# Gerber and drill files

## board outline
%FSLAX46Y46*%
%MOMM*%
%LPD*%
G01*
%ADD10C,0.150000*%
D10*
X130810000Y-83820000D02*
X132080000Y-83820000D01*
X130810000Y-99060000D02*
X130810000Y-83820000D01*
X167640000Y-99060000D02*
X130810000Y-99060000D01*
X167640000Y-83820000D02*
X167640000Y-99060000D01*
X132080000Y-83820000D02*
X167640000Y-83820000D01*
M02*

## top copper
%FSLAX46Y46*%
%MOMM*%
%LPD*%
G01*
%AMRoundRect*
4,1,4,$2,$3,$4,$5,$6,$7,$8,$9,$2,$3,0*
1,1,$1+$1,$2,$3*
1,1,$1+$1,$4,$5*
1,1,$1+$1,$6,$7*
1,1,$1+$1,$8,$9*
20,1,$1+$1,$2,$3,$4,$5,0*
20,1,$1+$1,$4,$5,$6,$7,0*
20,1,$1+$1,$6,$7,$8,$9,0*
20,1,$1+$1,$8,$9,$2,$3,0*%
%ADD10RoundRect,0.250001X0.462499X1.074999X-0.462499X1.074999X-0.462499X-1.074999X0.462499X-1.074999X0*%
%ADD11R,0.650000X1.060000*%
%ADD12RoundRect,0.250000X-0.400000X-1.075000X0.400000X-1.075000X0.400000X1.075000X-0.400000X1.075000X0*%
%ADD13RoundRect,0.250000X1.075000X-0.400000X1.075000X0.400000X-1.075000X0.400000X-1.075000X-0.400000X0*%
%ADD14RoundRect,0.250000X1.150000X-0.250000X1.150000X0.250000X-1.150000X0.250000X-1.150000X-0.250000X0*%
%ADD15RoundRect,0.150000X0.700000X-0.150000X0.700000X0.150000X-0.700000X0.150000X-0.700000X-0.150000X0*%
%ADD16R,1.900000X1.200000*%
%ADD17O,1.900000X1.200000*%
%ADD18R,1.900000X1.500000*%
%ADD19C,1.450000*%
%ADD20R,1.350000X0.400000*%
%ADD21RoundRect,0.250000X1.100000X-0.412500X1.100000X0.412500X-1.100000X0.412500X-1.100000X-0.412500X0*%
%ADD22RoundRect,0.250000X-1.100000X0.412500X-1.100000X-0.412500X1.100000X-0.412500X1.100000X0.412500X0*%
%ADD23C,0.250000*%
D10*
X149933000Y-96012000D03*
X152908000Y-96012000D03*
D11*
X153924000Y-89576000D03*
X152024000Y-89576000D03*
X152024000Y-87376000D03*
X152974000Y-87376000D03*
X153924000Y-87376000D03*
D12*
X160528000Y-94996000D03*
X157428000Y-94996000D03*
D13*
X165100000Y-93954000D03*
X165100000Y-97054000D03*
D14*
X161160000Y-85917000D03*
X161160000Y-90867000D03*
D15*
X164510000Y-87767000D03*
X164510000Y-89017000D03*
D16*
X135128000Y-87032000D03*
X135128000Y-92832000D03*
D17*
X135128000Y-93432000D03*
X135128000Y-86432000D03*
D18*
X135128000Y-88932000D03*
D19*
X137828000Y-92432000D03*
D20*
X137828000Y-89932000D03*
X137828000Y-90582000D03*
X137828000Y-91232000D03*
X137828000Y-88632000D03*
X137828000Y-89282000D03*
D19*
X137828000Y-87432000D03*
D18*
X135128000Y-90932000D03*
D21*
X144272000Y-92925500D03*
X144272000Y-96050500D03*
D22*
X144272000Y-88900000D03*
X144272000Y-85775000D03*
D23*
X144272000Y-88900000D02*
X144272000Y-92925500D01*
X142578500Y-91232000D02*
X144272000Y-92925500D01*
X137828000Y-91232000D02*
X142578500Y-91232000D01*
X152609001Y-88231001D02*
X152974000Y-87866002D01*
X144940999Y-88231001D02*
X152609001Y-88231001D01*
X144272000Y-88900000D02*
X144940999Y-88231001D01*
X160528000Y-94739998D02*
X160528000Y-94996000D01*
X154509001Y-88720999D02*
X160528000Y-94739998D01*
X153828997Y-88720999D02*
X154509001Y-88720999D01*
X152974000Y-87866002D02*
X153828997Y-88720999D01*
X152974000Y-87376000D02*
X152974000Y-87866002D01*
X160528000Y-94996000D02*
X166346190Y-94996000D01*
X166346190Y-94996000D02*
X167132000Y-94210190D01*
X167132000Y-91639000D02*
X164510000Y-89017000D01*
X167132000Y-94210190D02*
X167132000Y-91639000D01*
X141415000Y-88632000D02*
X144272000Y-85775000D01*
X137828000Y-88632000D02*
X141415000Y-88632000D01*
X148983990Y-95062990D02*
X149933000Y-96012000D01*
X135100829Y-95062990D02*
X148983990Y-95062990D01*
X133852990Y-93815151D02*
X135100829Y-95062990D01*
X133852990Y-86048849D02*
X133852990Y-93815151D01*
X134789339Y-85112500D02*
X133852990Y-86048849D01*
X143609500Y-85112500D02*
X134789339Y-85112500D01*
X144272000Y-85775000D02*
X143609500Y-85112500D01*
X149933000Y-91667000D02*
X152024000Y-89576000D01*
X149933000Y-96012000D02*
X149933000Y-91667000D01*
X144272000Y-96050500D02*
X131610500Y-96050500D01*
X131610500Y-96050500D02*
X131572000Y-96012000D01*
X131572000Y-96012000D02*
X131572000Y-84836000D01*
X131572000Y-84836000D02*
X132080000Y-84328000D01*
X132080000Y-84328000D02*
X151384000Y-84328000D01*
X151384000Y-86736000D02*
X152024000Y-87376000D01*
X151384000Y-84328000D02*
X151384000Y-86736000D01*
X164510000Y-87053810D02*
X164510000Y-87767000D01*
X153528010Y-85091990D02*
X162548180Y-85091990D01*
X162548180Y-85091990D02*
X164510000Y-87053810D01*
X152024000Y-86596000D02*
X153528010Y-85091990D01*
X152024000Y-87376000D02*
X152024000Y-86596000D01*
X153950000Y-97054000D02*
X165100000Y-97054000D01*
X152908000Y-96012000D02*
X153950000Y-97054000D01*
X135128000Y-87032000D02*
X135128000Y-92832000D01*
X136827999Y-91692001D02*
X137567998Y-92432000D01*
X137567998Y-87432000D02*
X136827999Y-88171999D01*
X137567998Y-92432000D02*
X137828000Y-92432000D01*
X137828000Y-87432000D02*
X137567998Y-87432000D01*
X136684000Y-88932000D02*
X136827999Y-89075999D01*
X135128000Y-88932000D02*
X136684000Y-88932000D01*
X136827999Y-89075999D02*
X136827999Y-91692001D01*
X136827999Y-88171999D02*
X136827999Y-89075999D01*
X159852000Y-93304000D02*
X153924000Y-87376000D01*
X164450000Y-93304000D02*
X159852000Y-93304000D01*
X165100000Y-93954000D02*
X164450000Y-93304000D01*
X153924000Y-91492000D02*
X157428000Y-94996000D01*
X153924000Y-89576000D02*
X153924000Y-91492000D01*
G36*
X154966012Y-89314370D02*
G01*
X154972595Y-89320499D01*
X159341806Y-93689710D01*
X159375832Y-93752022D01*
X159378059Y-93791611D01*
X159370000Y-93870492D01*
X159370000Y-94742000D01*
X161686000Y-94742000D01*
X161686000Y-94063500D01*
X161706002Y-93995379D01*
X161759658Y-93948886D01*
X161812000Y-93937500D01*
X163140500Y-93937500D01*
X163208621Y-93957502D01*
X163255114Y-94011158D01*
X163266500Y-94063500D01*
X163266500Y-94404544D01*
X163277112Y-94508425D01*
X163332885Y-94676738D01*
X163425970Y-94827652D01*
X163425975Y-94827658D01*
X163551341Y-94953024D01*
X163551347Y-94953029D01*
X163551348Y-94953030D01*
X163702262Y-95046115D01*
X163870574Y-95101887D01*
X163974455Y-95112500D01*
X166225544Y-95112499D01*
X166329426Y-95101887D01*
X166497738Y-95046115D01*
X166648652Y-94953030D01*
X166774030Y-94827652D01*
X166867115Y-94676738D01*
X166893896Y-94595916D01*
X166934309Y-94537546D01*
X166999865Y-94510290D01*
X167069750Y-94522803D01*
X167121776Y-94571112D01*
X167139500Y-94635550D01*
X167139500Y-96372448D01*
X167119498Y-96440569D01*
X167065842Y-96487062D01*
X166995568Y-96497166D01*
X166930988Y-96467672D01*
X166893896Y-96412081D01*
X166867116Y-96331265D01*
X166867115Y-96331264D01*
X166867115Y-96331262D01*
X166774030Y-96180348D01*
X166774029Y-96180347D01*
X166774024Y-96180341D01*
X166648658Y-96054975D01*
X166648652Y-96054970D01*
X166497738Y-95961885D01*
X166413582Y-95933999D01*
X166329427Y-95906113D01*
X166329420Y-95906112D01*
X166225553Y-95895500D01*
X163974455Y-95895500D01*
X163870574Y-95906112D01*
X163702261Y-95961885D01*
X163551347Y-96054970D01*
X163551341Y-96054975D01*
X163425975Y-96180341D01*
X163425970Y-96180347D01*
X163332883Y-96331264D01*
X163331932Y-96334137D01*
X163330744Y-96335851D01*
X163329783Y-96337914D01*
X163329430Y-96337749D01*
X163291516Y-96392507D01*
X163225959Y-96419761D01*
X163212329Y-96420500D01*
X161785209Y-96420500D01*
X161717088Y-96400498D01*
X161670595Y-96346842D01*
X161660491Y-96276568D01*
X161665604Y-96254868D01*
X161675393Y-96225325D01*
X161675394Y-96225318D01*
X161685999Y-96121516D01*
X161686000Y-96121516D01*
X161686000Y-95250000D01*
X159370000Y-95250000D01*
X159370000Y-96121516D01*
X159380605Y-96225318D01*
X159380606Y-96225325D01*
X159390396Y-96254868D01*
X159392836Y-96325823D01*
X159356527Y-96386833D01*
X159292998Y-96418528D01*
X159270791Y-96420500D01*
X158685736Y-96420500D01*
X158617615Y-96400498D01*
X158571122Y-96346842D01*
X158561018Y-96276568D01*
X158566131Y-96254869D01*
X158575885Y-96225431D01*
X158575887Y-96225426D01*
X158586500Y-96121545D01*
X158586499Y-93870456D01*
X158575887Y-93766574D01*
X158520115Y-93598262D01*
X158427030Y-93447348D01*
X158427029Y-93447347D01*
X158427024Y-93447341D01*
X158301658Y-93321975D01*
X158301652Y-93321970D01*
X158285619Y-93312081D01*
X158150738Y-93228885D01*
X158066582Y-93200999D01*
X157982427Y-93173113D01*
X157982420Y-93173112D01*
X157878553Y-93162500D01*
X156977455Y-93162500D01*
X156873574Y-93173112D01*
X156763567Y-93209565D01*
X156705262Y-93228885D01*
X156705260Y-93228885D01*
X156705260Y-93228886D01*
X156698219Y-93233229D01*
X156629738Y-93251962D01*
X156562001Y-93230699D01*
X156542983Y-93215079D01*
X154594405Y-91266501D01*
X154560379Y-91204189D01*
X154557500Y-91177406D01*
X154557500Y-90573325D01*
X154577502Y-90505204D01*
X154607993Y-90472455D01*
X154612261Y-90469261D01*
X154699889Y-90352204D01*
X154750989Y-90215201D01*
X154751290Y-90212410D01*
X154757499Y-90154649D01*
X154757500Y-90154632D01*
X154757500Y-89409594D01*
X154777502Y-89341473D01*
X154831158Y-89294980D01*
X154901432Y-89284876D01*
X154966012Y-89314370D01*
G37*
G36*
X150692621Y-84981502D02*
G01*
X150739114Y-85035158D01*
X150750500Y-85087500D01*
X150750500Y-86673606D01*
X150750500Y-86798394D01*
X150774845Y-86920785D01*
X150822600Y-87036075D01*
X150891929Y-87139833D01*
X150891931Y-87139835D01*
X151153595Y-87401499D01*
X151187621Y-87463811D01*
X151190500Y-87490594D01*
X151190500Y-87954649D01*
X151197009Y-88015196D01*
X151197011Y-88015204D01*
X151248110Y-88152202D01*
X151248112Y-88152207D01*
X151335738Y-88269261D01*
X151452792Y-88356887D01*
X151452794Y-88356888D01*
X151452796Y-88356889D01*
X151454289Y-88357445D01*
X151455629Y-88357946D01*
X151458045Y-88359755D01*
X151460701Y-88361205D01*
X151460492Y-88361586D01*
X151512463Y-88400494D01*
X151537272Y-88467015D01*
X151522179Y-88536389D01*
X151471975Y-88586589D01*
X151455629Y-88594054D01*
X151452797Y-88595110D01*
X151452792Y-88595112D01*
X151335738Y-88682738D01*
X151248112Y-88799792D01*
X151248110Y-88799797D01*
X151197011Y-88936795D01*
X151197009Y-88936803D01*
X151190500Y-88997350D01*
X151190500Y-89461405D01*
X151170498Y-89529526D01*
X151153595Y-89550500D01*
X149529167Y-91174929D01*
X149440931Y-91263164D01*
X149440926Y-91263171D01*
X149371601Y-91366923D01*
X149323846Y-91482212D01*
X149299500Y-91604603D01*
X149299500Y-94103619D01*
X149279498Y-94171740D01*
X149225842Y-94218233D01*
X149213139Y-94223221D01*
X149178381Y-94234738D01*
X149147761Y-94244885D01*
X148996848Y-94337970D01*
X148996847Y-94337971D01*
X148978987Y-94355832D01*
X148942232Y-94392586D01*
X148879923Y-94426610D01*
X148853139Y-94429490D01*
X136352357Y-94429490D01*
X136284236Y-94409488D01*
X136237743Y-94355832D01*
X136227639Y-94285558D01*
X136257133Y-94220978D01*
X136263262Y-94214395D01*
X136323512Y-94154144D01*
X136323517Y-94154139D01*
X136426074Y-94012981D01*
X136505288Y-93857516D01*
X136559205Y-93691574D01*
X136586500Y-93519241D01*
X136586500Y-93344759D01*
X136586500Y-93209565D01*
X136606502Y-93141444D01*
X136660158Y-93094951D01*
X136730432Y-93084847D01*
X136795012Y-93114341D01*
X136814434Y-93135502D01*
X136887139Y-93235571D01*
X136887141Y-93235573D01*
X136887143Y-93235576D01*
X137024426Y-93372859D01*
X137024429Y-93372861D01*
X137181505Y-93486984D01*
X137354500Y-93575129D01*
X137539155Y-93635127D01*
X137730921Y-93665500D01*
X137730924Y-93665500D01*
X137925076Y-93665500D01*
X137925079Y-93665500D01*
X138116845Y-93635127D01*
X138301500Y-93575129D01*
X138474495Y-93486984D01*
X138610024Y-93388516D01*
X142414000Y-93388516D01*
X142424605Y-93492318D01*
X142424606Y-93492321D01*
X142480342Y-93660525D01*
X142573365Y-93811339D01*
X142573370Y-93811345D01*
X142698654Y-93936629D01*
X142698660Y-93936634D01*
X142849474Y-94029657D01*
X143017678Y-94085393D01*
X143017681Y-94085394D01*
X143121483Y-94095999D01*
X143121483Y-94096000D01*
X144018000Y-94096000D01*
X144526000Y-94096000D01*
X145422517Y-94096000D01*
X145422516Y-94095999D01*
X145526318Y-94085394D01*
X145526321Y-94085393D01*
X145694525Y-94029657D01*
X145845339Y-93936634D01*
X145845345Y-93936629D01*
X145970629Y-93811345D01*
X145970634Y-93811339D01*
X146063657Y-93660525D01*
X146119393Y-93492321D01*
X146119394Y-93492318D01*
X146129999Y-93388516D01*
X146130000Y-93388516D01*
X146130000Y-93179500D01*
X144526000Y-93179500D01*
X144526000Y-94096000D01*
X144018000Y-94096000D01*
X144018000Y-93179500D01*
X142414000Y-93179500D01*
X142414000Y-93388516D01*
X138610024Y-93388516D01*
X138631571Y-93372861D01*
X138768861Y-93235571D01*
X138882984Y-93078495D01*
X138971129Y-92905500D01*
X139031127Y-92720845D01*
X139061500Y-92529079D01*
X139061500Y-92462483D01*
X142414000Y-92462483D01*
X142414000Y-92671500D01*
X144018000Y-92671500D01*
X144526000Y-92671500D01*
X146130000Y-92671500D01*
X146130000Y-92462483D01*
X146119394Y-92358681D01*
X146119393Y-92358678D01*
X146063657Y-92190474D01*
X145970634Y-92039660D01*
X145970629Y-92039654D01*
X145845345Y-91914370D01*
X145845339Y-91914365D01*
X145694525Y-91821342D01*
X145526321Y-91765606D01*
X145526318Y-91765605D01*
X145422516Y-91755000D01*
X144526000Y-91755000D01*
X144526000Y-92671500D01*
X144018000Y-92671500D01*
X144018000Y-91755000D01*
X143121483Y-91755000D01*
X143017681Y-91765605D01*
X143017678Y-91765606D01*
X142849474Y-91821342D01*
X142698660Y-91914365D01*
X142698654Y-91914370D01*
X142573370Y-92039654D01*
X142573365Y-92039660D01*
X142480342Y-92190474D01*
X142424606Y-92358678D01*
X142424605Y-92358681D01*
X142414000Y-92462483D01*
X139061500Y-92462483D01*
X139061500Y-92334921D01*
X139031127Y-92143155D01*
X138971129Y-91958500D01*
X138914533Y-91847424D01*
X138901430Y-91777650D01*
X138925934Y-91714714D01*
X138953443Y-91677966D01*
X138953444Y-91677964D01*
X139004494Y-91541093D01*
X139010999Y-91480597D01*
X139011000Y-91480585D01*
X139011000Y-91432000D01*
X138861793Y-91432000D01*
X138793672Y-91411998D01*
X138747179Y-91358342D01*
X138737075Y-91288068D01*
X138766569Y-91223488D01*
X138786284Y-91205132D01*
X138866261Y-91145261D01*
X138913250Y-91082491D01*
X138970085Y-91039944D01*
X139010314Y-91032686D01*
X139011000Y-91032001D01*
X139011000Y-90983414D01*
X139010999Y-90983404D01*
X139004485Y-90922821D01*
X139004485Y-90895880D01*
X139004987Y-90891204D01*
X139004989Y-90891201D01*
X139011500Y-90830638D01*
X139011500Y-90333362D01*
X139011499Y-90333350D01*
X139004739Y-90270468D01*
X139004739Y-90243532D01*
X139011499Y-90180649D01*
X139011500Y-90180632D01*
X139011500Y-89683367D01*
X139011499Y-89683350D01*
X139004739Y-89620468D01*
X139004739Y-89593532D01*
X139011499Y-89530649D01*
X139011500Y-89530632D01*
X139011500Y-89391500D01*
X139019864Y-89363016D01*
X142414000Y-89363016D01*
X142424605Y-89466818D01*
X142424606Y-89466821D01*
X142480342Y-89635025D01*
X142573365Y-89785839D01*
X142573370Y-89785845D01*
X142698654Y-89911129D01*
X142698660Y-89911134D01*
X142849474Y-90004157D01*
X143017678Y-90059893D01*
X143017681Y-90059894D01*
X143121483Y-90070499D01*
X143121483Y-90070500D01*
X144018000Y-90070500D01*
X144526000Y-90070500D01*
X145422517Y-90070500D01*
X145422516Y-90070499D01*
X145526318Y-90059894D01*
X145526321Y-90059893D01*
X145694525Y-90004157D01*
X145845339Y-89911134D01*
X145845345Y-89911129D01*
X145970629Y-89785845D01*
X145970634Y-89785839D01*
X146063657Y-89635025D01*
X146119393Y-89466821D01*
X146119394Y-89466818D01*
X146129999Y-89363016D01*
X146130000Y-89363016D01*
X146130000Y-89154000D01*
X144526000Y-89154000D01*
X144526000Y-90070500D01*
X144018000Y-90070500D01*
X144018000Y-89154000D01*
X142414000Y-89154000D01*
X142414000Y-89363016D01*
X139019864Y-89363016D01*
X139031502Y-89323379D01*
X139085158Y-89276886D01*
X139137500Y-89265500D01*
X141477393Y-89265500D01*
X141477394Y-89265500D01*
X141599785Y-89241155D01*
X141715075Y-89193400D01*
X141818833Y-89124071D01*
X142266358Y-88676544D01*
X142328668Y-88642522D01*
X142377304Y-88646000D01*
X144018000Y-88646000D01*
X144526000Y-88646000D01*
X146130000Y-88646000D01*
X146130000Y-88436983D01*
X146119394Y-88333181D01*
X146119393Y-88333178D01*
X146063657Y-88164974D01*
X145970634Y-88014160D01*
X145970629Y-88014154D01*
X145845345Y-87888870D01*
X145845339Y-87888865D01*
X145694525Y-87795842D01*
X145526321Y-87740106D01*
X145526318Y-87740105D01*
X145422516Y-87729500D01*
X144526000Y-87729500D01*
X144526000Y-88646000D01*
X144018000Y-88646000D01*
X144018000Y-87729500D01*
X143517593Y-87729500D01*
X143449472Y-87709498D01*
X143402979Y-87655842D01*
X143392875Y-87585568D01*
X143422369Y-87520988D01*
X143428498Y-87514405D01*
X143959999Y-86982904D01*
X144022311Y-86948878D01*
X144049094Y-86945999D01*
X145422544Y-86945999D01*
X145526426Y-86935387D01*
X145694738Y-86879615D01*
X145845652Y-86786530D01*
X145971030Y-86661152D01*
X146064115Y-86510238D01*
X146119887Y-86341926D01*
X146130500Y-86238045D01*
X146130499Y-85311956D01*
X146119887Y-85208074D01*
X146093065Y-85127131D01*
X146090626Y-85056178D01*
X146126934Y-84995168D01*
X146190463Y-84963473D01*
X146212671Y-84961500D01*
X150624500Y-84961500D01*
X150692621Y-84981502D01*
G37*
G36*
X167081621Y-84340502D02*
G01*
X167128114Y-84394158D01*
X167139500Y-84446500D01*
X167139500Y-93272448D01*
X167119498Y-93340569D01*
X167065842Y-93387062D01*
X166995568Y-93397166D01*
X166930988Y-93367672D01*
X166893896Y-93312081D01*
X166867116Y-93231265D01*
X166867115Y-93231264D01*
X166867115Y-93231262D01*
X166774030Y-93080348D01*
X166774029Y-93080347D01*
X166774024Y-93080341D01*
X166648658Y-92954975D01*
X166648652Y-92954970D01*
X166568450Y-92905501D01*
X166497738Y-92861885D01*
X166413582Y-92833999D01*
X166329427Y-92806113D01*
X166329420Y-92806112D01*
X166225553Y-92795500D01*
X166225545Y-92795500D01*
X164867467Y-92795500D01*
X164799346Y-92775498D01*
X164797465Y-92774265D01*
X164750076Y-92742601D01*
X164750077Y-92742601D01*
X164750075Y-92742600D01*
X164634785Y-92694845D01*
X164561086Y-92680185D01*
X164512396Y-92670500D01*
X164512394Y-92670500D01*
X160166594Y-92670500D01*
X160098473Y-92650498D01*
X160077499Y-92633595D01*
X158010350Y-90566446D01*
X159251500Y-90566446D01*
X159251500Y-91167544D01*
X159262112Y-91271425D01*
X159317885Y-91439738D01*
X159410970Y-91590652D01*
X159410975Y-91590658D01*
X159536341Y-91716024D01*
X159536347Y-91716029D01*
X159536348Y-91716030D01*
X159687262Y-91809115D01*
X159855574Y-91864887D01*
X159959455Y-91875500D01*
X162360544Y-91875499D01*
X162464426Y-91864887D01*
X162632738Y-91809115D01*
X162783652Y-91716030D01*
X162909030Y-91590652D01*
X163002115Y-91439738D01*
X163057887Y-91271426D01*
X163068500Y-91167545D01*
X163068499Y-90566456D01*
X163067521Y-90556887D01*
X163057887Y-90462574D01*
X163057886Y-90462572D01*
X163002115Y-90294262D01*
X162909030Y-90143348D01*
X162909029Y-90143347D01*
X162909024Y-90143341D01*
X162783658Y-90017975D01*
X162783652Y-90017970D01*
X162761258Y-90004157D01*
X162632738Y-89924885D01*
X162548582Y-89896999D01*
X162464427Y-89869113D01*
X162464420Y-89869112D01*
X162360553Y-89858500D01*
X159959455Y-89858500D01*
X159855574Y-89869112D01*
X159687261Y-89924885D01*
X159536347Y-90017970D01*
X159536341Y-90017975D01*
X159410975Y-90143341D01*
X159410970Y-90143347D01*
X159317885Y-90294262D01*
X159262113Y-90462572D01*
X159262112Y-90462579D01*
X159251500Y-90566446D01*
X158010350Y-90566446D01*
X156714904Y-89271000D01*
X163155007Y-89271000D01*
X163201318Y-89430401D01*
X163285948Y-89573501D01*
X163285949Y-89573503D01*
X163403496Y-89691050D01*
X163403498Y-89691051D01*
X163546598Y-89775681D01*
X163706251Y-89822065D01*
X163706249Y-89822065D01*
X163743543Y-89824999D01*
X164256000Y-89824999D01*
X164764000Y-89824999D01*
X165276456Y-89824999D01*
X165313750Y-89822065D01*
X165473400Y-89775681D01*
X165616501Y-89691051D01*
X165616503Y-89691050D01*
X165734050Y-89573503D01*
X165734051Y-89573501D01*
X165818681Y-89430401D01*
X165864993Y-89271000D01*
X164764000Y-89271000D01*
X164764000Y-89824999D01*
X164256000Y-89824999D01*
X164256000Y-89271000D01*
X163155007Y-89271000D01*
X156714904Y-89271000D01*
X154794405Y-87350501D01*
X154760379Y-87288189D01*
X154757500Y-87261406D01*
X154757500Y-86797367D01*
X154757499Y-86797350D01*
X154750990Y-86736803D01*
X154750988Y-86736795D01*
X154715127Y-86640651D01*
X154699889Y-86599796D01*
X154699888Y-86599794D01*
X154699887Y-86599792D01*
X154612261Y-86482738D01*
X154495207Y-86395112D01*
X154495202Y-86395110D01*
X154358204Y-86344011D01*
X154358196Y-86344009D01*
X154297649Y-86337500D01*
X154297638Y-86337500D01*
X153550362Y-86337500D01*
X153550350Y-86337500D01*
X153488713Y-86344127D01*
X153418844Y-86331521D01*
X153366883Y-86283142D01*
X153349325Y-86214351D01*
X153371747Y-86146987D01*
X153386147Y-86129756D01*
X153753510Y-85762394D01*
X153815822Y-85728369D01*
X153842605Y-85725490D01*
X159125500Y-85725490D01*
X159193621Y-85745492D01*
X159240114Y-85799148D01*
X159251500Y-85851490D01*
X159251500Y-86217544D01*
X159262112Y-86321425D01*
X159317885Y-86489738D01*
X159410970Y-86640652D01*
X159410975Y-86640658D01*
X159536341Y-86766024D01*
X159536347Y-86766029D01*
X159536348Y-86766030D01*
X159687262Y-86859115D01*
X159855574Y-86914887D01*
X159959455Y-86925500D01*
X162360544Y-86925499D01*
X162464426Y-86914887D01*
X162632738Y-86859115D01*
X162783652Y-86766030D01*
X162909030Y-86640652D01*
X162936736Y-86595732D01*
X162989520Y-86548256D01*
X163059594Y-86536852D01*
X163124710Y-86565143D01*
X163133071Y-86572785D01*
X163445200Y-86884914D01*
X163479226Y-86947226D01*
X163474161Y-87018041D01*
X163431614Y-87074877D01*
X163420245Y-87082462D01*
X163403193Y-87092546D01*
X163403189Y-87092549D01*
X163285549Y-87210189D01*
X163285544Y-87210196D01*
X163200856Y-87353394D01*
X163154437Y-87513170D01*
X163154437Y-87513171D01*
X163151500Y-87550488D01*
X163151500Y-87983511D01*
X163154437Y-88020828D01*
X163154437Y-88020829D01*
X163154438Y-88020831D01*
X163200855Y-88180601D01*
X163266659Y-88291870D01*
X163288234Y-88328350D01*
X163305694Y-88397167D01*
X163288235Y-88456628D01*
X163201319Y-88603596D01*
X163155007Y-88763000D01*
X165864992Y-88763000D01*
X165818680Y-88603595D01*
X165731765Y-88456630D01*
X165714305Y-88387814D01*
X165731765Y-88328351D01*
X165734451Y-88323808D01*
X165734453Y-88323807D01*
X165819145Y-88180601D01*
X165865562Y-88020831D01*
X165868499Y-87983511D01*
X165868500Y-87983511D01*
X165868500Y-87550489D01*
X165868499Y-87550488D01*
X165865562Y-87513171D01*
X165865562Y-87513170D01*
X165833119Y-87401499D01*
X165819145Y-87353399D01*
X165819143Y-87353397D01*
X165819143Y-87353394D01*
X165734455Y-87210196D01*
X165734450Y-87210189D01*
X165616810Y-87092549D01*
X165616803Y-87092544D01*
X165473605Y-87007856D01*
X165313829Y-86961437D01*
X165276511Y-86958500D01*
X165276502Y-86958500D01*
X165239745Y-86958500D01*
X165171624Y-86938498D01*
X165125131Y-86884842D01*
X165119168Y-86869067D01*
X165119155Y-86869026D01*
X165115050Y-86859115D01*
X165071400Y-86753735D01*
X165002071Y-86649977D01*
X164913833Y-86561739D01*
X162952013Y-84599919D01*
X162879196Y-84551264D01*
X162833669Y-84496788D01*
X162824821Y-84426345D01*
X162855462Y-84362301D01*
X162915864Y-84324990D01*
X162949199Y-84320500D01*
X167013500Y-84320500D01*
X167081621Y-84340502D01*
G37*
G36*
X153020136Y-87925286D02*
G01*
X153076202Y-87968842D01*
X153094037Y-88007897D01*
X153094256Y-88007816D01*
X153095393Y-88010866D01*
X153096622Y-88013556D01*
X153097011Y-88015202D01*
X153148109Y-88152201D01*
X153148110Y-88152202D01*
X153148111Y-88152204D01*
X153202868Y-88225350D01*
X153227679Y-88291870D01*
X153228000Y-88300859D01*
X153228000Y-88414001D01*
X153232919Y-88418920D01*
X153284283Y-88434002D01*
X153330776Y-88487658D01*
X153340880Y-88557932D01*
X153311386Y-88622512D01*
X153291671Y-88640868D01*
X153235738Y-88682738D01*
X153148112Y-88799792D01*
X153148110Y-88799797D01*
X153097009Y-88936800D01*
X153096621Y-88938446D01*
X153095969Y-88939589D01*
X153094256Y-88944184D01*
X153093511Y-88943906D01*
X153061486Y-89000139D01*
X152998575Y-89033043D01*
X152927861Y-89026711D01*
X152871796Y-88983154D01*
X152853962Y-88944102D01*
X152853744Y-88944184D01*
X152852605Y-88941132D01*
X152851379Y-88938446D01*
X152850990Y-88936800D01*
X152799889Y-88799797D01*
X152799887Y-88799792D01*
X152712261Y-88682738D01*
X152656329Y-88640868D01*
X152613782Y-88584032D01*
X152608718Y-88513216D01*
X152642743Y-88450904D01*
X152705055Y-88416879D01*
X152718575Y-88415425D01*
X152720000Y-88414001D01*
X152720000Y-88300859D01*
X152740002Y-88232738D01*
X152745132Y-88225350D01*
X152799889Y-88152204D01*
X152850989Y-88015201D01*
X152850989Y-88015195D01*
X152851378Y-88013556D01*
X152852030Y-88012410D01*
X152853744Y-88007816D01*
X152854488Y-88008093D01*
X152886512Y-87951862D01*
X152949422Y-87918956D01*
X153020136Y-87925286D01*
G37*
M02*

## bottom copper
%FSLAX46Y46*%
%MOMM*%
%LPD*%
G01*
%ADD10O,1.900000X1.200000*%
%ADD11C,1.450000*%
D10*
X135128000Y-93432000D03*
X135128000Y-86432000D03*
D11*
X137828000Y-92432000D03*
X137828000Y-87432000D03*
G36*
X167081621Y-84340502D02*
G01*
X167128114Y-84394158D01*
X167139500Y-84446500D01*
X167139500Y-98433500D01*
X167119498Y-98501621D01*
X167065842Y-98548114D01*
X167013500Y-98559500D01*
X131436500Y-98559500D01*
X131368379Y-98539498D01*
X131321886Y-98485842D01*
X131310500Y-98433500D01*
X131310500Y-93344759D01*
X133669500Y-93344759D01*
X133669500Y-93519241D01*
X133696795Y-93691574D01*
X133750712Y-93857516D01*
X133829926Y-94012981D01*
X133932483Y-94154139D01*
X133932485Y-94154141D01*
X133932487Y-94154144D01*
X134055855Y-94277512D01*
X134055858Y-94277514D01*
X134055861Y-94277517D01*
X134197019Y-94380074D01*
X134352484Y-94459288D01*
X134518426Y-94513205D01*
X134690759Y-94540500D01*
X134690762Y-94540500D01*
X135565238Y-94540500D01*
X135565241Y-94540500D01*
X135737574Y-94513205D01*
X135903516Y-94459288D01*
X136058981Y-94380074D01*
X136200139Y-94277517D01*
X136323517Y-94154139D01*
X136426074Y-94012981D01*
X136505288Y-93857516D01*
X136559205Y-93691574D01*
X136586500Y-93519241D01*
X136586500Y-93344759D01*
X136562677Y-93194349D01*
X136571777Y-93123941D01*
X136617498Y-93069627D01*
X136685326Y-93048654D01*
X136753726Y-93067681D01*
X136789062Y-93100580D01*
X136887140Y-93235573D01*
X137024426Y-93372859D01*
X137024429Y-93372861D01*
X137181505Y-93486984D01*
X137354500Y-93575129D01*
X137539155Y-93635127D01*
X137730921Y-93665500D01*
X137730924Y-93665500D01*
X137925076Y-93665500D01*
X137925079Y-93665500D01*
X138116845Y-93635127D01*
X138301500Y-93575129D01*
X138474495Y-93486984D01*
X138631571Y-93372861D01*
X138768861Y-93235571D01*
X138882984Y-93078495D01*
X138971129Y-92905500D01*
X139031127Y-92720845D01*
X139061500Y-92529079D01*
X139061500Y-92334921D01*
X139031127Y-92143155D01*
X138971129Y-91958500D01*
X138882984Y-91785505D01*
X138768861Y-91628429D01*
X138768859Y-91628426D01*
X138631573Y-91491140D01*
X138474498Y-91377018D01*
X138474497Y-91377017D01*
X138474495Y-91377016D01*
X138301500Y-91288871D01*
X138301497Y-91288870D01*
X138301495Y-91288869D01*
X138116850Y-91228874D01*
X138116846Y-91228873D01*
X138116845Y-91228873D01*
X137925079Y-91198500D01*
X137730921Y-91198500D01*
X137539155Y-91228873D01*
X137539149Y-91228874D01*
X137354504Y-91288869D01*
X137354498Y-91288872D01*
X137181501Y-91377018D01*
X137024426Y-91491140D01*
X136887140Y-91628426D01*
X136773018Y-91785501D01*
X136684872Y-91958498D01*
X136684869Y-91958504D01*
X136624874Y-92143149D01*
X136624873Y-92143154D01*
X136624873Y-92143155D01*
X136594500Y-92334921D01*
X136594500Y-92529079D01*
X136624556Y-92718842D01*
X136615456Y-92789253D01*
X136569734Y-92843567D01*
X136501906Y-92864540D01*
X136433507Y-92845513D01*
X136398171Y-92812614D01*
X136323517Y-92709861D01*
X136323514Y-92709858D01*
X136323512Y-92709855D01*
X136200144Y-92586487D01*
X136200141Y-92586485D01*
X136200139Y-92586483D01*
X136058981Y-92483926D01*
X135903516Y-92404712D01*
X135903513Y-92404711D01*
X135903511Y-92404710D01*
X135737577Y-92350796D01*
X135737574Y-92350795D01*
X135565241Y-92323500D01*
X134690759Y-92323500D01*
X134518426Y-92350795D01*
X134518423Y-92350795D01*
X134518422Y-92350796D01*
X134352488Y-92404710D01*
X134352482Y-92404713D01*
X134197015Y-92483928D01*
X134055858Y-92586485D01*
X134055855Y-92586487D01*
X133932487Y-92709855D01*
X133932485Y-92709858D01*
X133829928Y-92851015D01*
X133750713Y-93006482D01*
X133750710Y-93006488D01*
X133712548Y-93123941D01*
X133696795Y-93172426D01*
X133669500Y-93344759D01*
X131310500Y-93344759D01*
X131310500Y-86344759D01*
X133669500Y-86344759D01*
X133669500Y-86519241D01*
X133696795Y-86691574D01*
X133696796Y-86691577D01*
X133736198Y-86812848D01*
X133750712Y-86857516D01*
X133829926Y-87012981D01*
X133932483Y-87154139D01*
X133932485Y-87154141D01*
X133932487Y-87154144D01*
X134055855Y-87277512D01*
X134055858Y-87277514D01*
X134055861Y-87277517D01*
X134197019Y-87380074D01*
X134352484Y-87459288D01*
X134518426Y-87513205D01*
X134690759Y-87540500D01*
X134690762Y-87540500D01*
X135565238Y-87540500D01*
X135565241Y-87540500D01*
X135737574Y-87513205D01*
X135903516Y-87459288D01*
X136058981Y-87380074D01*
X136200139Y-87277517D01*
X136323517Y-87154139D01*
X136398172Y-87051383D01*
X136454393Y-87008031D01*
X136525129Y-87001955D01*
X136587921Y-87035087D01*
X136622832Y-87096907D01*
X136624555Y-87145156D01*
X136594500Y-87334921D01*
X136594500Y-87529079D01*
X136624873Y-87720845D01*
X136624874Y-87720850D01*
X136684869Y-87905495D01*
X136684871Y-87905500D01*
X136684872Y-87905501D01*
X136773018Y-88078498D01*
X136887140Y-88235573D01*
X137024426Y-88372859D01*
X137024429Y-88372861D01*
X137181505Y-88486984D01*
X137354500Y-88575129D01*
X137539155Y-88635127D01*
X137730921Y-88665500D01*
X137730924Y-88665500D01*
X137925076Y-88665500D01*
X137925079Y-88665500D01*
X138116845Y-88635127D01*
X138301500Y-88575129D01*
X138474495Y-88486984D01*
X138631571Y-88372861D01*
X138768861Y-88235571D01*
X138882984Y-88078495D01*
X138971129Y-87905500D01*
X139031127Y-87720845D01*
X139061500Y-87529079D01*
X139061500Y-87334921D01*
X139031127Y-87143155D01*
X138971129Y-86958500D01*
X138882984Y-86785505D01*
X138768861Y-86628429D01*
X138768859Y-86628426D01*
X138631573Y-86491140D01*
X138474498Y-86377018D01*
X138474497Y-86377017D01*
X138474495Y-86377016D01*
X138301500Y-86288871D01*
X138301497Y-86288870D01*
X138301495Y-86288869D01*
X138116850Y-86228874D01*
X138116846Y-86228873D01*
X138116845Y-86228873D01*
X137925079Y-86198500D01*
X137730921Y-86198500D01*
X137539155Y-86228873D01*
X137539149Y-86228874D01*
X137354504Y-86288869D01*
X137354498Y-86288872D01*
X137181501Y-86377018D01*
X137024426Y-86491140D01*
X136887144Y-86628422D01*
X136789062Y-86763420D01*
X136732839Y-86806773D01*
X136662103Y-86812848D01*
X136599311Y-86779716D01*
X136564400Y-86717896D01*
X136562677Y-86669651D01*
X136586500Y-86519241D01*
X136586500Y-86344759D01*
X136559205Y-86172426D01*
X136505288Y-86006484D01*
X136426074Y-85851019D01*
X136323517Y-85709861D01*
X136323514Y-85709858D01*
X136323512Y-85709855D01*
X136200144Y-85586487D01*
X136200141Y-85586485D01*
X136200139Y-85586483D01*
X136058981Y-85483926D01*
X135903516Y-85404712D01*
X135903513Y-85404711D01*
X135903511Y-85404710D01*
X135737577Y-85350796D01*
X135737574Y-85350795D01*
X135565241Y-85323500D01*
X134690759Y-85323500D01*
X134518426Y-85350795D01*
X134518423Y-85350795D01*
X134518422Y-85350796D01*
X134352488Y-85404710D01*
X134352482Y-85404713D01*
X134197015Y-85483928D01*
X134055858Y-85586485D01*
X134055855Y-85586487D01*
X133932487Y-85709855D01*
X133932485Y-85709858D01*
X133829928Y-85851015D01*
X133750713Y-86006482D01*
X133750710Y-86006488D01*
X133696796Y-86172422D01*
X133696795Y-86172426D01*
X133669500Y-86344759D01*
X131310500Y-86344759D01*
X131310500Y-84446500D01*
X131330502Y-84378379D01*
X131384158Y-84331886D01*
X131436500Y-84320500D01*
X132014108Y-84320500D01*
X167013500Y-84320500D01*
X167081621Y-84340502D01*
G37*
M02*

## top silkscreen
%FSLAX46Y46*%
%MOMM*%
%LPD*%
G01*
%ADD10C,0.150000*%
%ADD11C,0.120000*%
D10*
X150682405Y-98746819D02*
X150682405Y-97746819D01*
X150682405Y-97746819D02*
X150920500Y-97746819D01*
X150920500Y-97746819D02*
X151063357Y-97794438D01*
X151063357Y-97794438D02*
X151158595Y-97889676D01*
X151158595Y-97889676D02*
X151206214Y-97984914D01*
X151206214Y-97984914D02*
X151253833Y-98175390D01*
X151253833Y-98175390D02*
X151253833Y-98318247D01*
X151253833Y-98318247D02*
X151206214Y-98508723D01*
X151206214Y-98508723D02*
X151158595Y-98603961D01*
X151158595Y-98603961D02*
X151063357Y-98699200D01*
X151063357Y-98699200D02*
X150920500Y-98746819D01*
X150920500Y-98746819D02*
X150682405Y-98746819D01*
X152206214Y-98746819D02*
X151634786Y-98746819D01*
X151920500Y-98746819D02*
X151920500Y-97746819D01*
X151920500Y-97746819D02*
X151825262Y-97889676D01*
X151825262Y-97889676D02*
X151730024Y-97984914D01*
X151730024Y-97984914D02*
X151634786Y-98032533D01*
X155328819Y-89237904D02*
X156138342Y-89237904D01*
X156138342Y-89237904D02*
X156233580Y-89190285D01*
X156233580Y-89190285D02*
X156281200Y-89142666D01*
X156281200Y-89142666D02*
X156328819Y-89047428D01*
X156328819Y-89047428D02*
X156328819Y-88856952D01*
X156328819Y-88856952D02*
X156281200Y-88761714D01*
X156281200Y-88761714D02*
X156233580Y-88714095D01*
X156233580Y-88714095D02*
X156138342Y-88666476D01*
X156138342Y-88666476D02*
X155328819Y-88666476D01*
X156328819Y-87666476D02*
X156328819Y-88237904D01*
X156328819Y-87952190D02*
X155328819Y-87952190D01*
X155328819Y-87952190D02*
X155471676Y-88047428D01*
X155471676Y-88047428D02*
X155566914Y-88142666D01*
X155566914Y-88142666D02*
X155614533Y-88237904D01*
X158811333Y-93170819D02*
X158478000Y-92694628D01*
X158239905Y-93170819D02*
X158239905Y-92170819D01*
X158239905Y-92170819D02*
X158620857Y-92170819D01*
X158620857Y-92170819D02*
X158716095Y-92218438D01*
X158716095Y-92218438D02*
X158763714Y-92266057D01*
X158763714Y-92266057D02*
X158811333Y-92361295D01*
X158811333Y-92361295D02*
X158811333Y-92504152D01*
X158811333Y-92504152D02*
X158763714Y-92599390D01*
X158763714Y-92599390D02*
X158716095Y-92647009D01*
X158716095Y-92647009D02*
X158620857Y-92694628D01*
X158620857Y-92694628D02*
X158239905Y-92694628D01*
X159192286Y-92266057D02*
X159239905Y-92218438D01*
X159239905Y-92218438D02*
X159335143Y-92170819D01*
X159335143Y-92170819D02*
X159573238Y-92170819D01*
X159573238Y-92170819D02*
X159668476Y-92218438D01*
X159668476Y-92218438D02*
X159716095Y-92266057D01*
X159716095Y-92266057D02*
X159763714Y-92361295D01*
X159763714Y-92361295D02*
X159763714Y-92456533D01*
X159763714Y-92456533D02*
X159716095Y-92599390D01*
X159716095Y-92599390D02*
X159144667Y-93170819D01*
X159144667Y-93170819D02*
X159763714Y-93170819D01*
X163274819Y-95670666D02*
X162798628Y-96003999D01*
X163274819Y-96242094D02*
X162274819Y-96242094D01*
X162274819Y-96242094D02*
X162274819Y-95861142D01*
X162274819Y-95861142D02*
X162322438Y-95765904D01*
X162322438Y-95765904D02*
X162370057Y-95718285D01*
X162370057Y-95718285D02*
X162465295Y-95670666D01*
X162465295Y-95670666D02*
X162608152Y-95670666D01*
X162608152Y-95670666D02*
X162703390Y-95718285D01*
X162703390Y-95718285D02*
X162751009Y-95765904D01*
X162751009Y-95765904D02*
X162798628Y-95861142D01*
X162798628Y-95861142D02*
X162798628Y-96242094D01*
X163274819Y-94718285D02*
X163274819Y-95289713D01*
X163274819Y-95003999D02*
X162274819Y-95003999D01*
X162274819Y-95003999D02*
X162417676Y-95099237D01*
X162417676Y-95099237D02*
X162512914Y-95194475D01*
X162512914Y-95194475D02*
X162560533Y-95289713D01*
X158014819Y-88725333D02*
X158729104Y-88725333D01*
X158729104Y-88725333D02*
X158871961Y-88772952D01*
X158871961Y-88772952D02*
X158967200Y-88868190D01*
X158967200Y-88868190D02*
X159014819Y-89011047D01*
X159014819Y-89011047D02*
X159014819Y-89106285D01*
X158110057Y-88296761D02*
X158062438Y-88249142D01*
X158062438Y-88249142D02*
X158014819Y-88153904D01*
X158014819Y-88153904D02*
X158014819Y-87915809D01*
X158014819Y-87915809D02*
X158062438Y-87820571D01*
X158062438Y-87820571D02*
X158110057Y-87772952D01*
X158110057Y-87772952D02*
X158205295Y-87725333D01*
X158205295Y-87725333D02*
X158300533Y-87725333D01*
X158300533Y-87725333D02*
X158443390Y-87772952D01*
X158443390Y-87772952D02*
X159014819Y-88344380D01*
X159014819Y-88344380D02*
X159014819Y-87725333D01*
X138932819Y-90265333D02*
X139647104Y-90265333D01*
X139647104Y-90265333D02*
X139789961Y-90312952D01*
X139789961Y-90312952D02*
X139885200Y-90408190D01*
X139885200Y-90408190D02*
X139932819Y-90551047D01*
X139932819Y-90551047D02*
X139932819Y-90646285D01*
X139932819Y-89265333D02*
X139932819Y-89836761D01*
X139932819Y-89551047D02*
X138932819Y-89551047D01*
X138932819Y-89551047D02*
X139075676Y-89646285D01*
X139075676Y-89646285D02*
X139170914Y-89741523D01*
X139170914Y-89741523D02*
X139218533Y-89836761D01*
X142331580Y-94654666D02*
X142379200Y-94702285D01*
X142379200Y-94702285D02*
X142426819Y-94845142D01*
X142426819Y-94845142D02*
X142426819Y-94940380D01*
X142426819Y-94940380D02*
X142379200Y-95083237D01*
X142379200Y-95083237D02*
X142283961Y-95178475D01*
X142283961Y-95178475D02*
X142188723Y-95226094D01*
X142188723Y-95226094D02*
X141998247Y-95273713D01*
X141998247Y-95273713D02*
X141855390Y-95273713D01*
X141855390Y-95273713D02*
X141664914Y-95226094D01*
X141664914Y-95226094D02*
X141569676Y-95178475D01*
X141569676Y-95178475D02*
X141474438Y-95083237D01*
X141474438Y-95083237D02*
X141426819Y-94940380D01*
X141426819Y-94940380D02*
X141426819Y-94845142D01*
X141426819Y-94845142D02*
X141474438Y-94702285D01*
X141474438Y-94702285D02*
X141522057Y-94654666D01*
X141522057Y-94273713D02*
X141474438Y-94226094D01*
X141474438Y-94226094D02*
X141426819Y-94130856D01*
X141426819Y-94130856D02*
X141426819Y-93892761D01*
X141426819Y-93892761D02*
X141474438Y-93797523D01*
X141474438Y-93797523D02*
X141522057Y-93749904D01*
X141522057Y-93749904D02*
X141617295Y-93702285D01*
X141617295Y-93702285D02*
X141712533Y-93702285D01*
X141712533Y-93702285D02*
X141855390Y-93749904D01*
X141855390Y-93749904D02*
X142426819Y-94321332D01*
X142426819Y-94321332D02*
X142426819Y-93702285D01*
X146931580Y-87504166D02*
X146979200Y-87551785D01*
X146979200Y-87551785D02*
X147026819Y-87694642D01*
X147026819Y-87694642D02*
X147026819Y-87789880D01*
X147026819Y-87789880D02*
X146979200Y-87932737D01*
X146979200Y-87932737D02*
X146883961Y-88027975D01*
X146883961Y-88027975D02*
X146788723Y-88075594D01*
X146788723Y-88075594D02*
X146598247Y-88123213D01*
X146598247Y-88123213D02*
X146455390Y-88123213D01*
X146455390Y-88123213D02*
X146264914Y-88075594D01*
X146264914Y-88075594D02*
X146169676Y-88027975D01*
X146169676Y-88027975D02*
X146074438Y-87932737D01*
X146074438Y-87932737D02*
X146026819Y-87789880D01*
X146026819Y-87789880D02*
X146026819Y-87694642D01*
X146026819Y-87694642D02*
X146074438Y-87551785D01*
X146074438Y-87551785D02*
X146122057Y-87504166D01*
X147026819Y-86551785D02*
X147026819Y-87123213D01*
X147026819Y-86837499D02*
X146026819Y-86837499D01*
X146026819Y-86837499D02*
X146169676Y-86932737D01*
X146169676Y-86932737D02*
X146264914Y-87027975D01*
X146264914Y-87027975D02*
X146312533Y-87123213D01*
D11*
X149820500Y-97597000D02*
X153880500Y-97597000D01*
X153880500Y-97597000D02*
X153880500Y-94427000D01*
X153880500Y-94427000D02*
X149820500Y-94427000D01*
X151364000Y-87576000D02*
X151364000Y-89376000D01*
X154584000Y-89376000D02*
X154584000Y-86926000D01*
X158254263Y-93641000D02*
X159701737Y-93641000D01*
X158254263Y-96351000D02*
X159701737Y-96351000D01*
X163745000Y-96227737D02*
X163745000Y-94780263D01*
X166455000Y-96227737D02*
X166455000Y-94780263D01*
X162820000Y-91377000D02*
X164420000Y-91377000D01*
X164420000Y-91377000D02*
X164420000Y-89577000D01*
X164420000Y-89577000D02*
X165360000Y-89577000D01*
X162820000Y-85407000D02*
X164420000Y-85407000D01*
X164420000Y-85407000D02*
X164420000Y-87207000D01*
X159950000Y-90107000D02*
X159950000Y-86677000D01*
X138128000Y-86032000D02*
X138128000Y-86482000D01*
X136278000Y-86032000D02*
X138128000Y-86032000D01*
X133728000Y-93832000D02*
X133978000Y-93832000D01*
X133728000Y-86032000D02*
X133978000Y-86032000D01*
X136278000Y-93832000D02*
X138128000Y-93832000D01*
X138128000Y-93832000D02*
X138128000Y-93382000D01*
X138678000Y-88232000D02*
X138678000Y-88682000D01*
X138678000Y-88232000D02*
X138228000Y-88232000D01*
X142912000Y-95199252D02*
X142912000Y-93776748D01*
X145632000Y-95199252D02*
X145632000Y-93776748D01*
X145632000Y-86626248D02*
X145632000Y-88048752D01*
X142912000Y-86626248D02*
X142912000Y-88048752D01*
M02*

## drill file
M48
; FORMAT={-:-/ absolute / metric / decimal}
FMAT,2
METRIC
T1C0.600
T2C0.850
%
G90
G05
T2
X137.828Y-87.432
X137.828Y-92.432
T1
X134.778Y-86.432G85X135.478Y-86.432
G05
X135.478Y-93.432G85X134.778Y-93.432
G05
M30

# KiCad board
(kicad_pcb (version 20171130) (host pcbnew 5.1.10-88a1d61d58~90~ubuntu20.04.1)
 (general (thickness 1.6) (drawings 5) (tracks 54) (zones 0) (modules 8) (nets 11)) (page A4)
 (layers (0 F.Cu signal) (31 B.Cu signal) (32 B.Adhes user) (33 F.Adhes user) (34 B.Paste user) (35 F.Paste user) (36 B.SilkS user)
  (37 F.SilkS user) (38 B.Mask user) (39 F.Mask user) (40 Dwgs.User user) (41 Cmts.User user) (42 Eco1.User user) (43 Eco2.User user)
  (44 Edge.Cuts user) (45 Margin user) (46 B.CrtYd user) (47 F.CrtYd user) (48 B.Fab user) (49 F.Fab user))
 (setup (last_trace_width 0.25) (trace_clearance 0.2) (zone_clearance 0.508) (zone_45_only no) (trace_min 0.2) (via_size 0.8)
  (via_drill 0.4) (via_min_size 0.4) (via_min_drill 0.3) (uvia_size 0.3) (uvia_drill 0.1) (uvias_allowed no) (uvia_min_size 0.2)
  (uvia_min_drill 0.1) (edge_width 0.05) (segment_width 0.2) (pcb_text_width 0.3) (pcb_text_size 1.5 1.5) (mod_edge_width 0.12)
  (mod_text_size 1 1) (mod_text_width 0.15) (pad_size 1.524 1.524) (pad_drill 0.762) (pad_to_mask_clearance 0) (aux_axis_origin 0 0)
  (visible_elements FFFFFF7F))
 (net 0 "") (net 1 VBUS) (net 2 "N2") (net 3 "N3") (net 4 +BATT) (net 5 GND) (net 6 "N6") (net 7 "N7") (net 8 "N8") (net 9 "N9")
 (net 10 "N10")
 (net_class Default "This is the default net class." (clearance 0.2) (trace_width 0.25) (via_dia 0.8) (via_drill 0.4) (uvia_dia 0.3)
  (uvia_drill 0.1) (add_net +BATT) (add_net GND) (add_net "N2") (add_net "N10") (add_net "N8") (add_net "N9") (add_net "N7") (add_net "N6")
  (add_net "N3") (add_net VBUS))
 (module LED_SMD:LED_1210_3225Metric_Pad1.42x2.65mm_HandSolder (layer F.Cu) (at 151.4205 96.012 180)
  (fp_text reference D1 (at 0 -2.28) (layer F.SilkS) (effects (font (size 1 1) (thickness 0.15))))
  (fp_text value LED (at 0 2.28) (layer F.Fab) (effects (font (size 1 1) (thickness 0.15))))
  (fp_line (start 1.6 -1.585) (end -2.46 -1.585) (layer F.SilkS) (width 0.12))
  (fp_line (start -2.46 -1.585) (end -2.46 1.585) (layer F.SilkS) (width 0.12))
  (fp_line (start -2.46 1.585) (end 1.6 1.585) (layer F.SilkS) (width 0.12))
  (pad 2 smd roundrect (at 1.4875 0 180) (size 1.425 2.65) (layers F.Cu F.Paste F.Mask) (roundrect_rratio 0.175439) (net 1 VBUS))
  (pad 1 smd roundrect (at -1.4875 0 180) (size 1.425 2.65) (layers F.Cu F.Paste F.Mask) (roundrect_rratio 0.175439) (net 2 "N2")))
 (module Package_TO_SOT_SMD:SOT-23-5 (layer F.Cu) (at 152.974 88.476 270)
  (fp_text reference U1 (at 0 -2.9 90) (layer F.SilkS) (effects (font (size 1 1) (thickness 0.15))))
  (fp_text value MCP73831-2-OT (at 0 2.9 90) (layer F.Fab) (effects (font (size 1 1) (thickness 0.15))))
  (fp_line (start -0.9 1.61) (end 0.9 1.61) (layer F.SilkS) (width 0.12))
  (fp_line (start 0.9 -1.61) (end -1.55 -1.61) (layer F.SilkS) (width 0.12))
  (pad 5 smd rect (at 1.1 -0.95 270) (size 1.06 0.65) (layers F.Cu F.Paste F.Mask) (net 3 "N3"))
  (pad 4 smd rect (at 1.1 0.95 270) (size 1.06 0.65) (layers F.Cu F.Paste F.Mask) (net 1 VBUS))
  (pad 3 smd rect (at -1.1 0.95 270) (size 1.06 0.65) (layers F.Cu F.Paste F.Mask) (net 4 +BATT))
  (pad 2 smd rect (at -1.1 0 270) (size 1.06 0.65) (layers F.Cu F.Paste F.Mask) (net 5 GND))
  (pad 1 smd rect (at -1.1 -0.95 270) (size 1.06 0.65) (layers F.Cu F.Paste F.Mask) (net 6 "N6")))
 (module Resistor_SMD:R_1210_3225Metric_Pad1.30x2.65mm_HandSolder (layer F.Cu) (at 158.978 94.996)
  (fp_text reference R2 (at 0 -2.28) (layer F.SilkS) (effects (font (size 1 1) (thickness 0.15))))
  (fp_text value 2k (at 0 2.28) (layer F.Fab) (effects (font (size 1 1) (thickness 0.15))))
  (fp_line (start -0.723737 -1.355) (end 0.723737 -1.355) (layer F.SilkS) (width 0.12))
  (fp_line (start -0.723737 1.355) (end 0.723737 1.355) (layer F.SilkS) (width 0.12))
  (pad 2 smd roundrect (at 1.55 0) (size 1.3 2.65) (layers F.Cu F.Paste F.Mask) (roundrect_rratio 0.192308) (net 5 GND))
  (pad 1 smd roundrect (at -1.55 0) (size 1.3 2.65) (layers F.Cu F.Paste F.Mask) (roundrect_rratio 0.192308) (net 3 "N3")))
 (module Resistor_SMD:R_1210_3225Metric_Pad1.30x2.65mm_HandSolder (layer F.Cu) (at 165.1 95.504 90)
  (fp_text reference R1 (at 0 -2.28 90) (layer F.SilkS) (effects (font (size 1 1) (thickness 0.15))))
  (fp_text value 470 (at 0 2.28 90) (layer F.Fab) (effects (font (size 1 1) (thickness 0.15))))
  (fp_line (start -0.723737 -1.355) (end 0.723737 -1.355) (layer F.SilkS) (width 0.12))
  (fp_line (start -0.723737 1.355) (end 0.723737 1.355) (layer F.SilkS) (width 0.12))
  (pad 2 smd roundrect (at 1.55 0 90) (size 1.3 2.65) (layers F.Cu F.Paste F.Mask) (roundrect_rratio 0.192308) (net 6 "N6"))
  (pad 1 smd roundrect (at -1.55 0 90) (size 1.3 2.65) (layers F.Cu F.Paste F.Mask) (roundrect_rratio 0.192308) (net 2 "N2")))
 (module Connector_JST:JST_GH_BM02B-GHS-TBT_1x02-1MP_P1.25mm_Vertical (layer F.Cu) (at 162.56 88.392 90)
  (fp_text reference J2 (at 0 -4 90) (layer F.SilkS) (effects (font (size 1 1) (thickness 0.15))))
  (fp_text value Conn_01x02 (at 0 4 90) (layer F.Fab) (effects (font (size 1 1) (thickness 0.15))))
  (fp_line (start -2.985 0.26) (end -2.985 1.86) (layer F.SilkS) (width 0.12))
  (fp_line (start -2.985 1.86) (end -1.185 1.86) (layer F.SilkS) (width 0.12))
  (fp_line (start -1.185 1.86) (end -1.185 2.8) (layer F.SilkS) (width 0.12))
  (fp_line (start 2.985 0.26) (end 2.985 1.86) (layer F.SilkS) (width 0.12))
  (fp_line (start 2.985 1.86) (end 1.185 1.86) (layer F.SilkS) (width 0.12))
  (fp_line (start -1.715 -2.61) (end 1.715 -2.61) (layer F.SilkS) (width 0.12))
  (pad MP smd roundrect (at 2.475 -1.4 90) (size 1 2.8) (layers F.Cu F.Paste F.Mask) (roundrect_rratio 0.25))
  (pad MP smd roundrect (at -2.475 -1.4 90) (size 1 2.8) (layers F.Cu F.Paste F.Mask) (roundrect_rratio 0.25))
  (pad 2 smd roundrect (at 0.625 1.95 90) (size 0.6 1.7) (layers F.Cu F.Paste F.Mask) (roundrect_rratio 0.25) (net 4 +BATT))
  (pad 1 smd roundrect (at -0.625 1.95 90) (size 0.6 1.7) (layers F.Cu F.Paste F.Mask) (roundrect_rratio 0.25) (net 5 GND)))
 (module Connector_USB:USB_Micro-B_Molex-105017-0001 (layer F.Cu) (at 136.3655 89.932 270)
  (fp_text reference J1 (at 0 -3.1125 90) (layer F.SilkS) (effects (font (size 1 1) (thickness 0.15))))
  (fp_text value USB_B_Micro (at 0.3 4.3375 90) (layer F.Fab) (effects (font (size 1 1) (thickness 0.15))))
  (fp_line (start -3.9 -1.7625) (end -3.45 -1.7625) (layer F.SilkS) (width 0.12))
  (fp_line (start -3.9 0.0875) (end -3.9 -1.7625) (layer F.SilkS) (width 0.12))
  (fp_line (start 3.9 2.6375) (end 3.9 2.3875) (layer F.SilkS) (width 0.12))
  (fp_line (start -3.9 2.6375) (end -3.9 2.3875) (layer F.SilkS) (width 0.12))
  (fp_line (start 3.9 0.0875) (end 3.9 -1.7625) (layer F.SilkS) (width 0.12))
  (fp_line (start 3.9 -1.7625) (end 3.45 -1.7625) (layer F.SilkS) (width 0.12))
  (fp_line (start -1.7 -2.3125) (end -1.25 -2.3125) (layer F.SilkS) (width 0.12))
  (fp_line (start -1.7 -2.3125) (end -1.7 -1.8625) (layer F.SilkS) (width 0.12))
  (pad 6 smd rect (at -2.9 1.2375 270) (size 1.2 1.9) (layers F.Cu F.Mask) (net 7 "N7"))
  (pad 6 smd rect (at 2.9 1.2375 270) (size 1.2 1.9) (layers F.Cu F.Mask) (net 7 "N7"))
  (pad 6 thru_hole oval (at 3.5 1.2375 270) (size 1.2 1.9) (drill oval 0.6 1.3) (layers *.Cu *.Mask) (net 7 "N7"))
  (pad 6 thru_hole oval (at -3.5 1.2375 90) (size 1.2 1.9) (drill oval 0.6 1.3) (layers *.Cu *.Mask) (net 7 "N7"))
  (pad 6 smd rect (at -1 1.2375 270) (size 1.5 1.9) (layers F.Cu F.Paste F.Mask) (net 7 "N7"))
  (pad 6 thru_hole circle (at 2.5 -1.4625 270) (size 1.45 1.45) (drill 0.85) (layers *.Cu *.Mask) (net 7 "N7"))
  (pad 3 smd rect (at 0 -1.4625 270) (size 0.4 1.35) (layers F.Cu F.Paste F.Mask) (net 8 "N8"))
  (pad 4 smd rect (at 0.65 -1.4625 270) (size 0.4 1.35) (layers F.Cu F.Paste F.Mask) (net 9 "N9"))
  (pad 5 smd rect (at 1.3 -1.4625 270) (size 0.4 1.35) (layers F.Cu F.Paste F.Mask) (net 5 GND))
  (pad 1 smd rect (at -1.3 -1.4625 270) (size 0.4 1.35) (layers F.Cu F.Paste F.Mask) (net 1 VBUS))
  (pad 2 smd rect (at -0.65 -1.4625 270) (size 0.4 1.35) (layers F.Cu F.Paste F.Mask) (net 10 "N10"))
  (pad 6 thru_hole circle (at -2.5 -1.4625 270) (size 1.45 1.45) (drill 0.85) (layers *.Cu *.Mask) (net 7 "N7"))
  (pad 6 smd rect (at 1 1.2375 270) (size 1.5 1.9) (layers F.Cu F.Paste F.Mask) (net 7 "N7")))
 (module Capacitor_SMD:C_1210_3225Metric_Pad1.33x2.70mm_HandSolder (layer F.Cu) (at 144.272 94.488 90)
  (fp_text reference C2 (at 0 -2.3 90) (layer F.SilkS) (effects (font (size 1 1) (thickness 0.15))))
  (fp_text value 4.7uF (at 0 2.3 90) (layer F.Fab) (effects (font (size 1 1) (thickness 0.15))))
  (fp_line (start -0.711252 -1.36) (end 0.711252 -1.36) (layer F.SilkS) (width 0.12))
  (fp_line (start -0.711252 1.36) (end 0.711252 1.36) (layer F.SilkS) (width 0.12))
  (pad 2 smd roundrect (at 1.5625 0 90) (size 1.325 2.7) (layers F.Cu F.Paste F.Mask) (roundrect_rratio 0.188679) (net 5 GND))
  (pad 1 smd roundrect (at -1.5625 0 90) (size 1.325 2.7) (layers F.Cu F.Paste F.Mask) (roundrect_rratio 0.188679) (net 4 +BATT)))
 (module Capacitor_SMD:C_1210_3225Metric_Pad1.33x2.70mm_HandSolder (layer F.Cu) (at 144.272 87.3375 270)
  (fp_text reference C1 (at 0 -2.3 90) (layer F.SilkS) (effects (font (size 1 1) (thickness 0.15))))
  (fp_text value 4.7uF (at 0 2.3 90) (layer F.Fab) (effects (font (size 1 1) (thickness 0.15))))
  (fp_line (start -0.711252 -1.36) (end 0.711252 -1.36) (layer F.SilkS) (width 0.12))
  (fp_line (start -0.711252 1.36) (end 0.711252 1.36) (layer F.SilkS) (width 0.12))
  (pad 2 smd roundrect (at 1.5625 0 270) (size 1.325 2.7) (layers F.Cu F.Paste F.Mask) (roundrect_rratio 0.188679) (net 5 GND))
  (pad 1 smd roundrect (at -1.5625 0 270) (size 1.325 2.7) (layers F.Cu F.Paste F.Mask) (roundrect_rratio 0.188679) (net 1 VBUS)))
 (gr_line (start 130.81 83.82) (end 132.08 83.82) (layer Edge.Cuts) (width 0.15))
 (gr_line (start 130.81 99.06) (end 130.81 83.82) (layer Edge.Cuts) (width 0.15))
 (gr_line (start 167.64 99.06) (end 130.81 99.06) (layer Edge.Cuts) (width 0.15))
 (gr_line (start 167.64 83.82) (end 167.64 99.06) (layer Edge.Cuts) (width 0.15))
 (gr_line (start 132.08 83.82) (end 167.64 83.82) (layer Edge.Cuts) (width 0.15))
 (segment (start 144.272 88.9) (end 144.272 92.9255) (width 0.25) (layer F.Cu) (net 5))
 (segment (start 142.5785 91.232) (end 144.272 92.9255) (width 0.25) (layer F.Cu) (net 5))
 (segment (start 137.828 91.232) (end 142.5785 91.232) (width 0.25) (layer F.Cu) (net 5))
 (segment (start 152.609001 88.231001) (end 152.974 87.866002) (width 0.25) (layer F.Cu) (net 5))
 (segment (start 144.940999 88.231001) (end 152.609001 88.231001) (width 0.25) (layer F.Cu) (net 5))
 (segment (start 144.272 88.9) (end 144.940999 88.231001) (width 0.25) (layer F.Cu) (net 5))
 (segment (start 160.528 94.739998) (end 160.528 94.996) (width 0.25) (layer F.Cu) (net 5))
 (segment (start 154.509001 88.720999) (end 160.528 94.739998) (width 0.25) (layer F.Cu) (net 5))
 (segment (start 153.828997 88.720999) (end 154.509001 88.720999) (width 0.25) (layer F.Cu) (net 5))
 (segment (start 152.974 87.866002) (end 153.828997 88.720999) (width 0.25) (layer F.Cu) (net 5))
 (segment (start 152.974 87.376) (end 152.974 87.866002) (width 0.25) (layer F.Cu) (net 5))
 (segment (start 160.528 94.996) (end 166.34619 94.996) (width 0.25) (layer F.Cu) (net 5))
 (segment (start 166.34619 94.996) (end 167.132 94.21019) (width 0.25) (layer F.Cu) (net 5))
 (segment (start 167.132 91.639) (end 164.51 89.017) (width 0.25) (layer F.Cu) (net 5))
 (segment (start 167.132 94.21019) (end 167.132 91.639) (width 0.25) (layer F.Cu) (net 5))
 (segment (start 141.415 88.632) (end 144.272 85.775) (width 0.25) (layer F.Cu) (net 1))
 (segment (start 137.828 88.632) (end 141.415 88.632) (width 0.25) (layer F.Cu) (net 1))
 (segment (start 148.98399 95.06299) (end 149.933 96.012) (width 0.25) (layer F.Cu) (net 1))
 (segment (start 135.100829 95.06299) (end 148.98399 95.06299) (width 0.25) (layer F.Cu) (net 1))
 (segment (start 133.85299 93.815151) (end 135.100829 95.06299) (width 0.25) (layer F.Cu) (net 1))
 (segment (start 133.85299 86.048849) (end 133.85299 93.815151) (width 0.25) (layer F.Cu) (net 1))
 (segment (start 134.789339 85.1125) (end 133.85299 86.048849) (width 0.25) (layer F.Cu) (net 1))
 (segment (start 143.6095 85.1125) (end 134.789339 85.1125) (width 0.25) (layer F.Cu) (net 1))
 (segment (start 144.272 85.775) (end 143.6095 85.1125) (width 0.25) (layer F.Cu) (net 1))
 (segment (start 149.933 91.667) (end 152.024 89.576) (width 0.25) (layer F.Cu) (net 1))
 (segment (start 149.933 96.012) (end 149.933 91.667) (width 0.25) (layer F.Cu) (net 1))
 (segment (start 144.272 96.0505) (end 131.6105 96.0505) (width 0.25) (layer F.Cu) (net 4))
 (segment (start 131.6105 96.0505) (end 131.572 96.012) (width 0.25) (layer F.Cu) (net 4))
 (segment (start 131.572 96.012) (end 131.572 84.836) (width 0.25) (layer F.Cu) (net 4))
 (segment (start 131.572 84.836) (end 132.08 84.328) (width 0.25) (layer F.Cu) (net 4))
 (segment (start 132.08 84.328) (end 151.384 84.328) (width 0.25) (layer F.Cu) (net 4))
 (segment (start 151.384 86.736) (end 152.024 87.376) (width 0.25) (layer F.Cu) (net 4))
 (segment (start 151.384 84.328) (end 151.384 86.736) (width 0.25) (layer F.Cu) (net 4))
 (segment (start 164.51 87.05381) (end 164.51 87.767) (width 0.25) (layer F.Cu) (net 4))
 (segment (start 153.52801 85.09199) (end 162.54818 85.09199) (width 0.25) (layer F.Cu) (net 4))
 (segment (start 162.54818 85.09199) (end 164.51 87.05381) (width 0.25) (layer F.Cu) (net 4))
 (segment (start 152.024 86.596) (end 153.52801 85.09199) (width 0.25) (layer F.Cu) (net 4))
 (segment (start 152.024 87.376) (end 152.024 86.596) (width 0.25) (layer F.Cu) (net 4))
 (segment (start 153.95 97.054) (end 165.1 97.054) (width 0.25) (layer F.Cu) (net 2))
 (segment (start 152.908 96.012) (end 153.95 97.054) (width 0.25) (layer F.Cu) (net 2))
 (segment (start 135.128 87.032) (end 135.128 92.832) (width 0.25) (layer F.Cu) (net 7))
 (segment (start 136.827999 91.692001) (end 137.567998 92.432) (width 0.25) (layer F.Cu) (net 7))
 (segment (start 137.567998 87.432) (end 136.827999 88.171999) (width 0.25) (layer F.Cu) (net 7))
 (segment (start 137.567998 92.432) (end 137.828 92.432) (width 0.25) (layer F.Cu) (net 7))
 (segment (start 137.828 87.432) (end 137.567998 87.432) (width 0.25) (layer F.Cu) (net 7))
 (segment (start 136.684 88.932) (end 136.827999 89.075999) (width 0.25) (layer F.Cu) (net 7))
 (segment (start 135.128 88.932) (end 136.684 88.932) (width 0.25) (layer F.Cu) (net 7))
 (segment (start 136.827999 89.075999) (end 136.827999 91.692001) (width 0.25) (layer F.Cu) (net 7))
 (segment (start 136.827999 88.171999) (end 136.827999 89.075999) (width 0.25) (layer F.Cu) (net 7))
 (segment (start 159.852 93.304) (end 153.924 87.376) (width 0.25) (layer F.Cu) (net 6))
 (segment (start 164.45 93.304) (end 159.852 93.304) (width 0.25) (layer F.Cu) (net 6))
 (segment (start 165.1 93.954) (end 164.45 93.304) (width 0.25) (layer F.Cu) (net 6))
 (segment (start 153.924 91.492) (end 157.428 94.996) (width 0.25) (layer F.Cu) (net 3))
 (segment (start 153.924 89.576) (end 153.924 91.492) (width 0.25) (layer F.Cu) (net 3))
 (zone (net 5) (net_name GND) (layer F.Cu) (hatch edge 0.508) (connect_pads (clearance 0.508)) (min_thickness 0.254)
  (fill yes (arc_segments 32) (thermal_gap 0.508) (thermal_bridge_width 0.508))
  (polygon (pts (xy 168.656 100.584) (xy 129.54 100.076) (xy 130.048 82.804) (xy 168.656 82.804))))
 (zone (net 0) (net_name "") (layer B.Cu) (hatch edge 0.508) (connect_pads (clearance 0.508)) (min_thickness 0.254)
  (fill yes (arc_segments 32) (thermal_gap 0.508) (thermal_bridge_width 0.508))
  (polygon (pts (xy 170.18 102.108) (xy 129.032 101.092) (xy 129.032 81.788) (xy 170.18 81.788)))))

